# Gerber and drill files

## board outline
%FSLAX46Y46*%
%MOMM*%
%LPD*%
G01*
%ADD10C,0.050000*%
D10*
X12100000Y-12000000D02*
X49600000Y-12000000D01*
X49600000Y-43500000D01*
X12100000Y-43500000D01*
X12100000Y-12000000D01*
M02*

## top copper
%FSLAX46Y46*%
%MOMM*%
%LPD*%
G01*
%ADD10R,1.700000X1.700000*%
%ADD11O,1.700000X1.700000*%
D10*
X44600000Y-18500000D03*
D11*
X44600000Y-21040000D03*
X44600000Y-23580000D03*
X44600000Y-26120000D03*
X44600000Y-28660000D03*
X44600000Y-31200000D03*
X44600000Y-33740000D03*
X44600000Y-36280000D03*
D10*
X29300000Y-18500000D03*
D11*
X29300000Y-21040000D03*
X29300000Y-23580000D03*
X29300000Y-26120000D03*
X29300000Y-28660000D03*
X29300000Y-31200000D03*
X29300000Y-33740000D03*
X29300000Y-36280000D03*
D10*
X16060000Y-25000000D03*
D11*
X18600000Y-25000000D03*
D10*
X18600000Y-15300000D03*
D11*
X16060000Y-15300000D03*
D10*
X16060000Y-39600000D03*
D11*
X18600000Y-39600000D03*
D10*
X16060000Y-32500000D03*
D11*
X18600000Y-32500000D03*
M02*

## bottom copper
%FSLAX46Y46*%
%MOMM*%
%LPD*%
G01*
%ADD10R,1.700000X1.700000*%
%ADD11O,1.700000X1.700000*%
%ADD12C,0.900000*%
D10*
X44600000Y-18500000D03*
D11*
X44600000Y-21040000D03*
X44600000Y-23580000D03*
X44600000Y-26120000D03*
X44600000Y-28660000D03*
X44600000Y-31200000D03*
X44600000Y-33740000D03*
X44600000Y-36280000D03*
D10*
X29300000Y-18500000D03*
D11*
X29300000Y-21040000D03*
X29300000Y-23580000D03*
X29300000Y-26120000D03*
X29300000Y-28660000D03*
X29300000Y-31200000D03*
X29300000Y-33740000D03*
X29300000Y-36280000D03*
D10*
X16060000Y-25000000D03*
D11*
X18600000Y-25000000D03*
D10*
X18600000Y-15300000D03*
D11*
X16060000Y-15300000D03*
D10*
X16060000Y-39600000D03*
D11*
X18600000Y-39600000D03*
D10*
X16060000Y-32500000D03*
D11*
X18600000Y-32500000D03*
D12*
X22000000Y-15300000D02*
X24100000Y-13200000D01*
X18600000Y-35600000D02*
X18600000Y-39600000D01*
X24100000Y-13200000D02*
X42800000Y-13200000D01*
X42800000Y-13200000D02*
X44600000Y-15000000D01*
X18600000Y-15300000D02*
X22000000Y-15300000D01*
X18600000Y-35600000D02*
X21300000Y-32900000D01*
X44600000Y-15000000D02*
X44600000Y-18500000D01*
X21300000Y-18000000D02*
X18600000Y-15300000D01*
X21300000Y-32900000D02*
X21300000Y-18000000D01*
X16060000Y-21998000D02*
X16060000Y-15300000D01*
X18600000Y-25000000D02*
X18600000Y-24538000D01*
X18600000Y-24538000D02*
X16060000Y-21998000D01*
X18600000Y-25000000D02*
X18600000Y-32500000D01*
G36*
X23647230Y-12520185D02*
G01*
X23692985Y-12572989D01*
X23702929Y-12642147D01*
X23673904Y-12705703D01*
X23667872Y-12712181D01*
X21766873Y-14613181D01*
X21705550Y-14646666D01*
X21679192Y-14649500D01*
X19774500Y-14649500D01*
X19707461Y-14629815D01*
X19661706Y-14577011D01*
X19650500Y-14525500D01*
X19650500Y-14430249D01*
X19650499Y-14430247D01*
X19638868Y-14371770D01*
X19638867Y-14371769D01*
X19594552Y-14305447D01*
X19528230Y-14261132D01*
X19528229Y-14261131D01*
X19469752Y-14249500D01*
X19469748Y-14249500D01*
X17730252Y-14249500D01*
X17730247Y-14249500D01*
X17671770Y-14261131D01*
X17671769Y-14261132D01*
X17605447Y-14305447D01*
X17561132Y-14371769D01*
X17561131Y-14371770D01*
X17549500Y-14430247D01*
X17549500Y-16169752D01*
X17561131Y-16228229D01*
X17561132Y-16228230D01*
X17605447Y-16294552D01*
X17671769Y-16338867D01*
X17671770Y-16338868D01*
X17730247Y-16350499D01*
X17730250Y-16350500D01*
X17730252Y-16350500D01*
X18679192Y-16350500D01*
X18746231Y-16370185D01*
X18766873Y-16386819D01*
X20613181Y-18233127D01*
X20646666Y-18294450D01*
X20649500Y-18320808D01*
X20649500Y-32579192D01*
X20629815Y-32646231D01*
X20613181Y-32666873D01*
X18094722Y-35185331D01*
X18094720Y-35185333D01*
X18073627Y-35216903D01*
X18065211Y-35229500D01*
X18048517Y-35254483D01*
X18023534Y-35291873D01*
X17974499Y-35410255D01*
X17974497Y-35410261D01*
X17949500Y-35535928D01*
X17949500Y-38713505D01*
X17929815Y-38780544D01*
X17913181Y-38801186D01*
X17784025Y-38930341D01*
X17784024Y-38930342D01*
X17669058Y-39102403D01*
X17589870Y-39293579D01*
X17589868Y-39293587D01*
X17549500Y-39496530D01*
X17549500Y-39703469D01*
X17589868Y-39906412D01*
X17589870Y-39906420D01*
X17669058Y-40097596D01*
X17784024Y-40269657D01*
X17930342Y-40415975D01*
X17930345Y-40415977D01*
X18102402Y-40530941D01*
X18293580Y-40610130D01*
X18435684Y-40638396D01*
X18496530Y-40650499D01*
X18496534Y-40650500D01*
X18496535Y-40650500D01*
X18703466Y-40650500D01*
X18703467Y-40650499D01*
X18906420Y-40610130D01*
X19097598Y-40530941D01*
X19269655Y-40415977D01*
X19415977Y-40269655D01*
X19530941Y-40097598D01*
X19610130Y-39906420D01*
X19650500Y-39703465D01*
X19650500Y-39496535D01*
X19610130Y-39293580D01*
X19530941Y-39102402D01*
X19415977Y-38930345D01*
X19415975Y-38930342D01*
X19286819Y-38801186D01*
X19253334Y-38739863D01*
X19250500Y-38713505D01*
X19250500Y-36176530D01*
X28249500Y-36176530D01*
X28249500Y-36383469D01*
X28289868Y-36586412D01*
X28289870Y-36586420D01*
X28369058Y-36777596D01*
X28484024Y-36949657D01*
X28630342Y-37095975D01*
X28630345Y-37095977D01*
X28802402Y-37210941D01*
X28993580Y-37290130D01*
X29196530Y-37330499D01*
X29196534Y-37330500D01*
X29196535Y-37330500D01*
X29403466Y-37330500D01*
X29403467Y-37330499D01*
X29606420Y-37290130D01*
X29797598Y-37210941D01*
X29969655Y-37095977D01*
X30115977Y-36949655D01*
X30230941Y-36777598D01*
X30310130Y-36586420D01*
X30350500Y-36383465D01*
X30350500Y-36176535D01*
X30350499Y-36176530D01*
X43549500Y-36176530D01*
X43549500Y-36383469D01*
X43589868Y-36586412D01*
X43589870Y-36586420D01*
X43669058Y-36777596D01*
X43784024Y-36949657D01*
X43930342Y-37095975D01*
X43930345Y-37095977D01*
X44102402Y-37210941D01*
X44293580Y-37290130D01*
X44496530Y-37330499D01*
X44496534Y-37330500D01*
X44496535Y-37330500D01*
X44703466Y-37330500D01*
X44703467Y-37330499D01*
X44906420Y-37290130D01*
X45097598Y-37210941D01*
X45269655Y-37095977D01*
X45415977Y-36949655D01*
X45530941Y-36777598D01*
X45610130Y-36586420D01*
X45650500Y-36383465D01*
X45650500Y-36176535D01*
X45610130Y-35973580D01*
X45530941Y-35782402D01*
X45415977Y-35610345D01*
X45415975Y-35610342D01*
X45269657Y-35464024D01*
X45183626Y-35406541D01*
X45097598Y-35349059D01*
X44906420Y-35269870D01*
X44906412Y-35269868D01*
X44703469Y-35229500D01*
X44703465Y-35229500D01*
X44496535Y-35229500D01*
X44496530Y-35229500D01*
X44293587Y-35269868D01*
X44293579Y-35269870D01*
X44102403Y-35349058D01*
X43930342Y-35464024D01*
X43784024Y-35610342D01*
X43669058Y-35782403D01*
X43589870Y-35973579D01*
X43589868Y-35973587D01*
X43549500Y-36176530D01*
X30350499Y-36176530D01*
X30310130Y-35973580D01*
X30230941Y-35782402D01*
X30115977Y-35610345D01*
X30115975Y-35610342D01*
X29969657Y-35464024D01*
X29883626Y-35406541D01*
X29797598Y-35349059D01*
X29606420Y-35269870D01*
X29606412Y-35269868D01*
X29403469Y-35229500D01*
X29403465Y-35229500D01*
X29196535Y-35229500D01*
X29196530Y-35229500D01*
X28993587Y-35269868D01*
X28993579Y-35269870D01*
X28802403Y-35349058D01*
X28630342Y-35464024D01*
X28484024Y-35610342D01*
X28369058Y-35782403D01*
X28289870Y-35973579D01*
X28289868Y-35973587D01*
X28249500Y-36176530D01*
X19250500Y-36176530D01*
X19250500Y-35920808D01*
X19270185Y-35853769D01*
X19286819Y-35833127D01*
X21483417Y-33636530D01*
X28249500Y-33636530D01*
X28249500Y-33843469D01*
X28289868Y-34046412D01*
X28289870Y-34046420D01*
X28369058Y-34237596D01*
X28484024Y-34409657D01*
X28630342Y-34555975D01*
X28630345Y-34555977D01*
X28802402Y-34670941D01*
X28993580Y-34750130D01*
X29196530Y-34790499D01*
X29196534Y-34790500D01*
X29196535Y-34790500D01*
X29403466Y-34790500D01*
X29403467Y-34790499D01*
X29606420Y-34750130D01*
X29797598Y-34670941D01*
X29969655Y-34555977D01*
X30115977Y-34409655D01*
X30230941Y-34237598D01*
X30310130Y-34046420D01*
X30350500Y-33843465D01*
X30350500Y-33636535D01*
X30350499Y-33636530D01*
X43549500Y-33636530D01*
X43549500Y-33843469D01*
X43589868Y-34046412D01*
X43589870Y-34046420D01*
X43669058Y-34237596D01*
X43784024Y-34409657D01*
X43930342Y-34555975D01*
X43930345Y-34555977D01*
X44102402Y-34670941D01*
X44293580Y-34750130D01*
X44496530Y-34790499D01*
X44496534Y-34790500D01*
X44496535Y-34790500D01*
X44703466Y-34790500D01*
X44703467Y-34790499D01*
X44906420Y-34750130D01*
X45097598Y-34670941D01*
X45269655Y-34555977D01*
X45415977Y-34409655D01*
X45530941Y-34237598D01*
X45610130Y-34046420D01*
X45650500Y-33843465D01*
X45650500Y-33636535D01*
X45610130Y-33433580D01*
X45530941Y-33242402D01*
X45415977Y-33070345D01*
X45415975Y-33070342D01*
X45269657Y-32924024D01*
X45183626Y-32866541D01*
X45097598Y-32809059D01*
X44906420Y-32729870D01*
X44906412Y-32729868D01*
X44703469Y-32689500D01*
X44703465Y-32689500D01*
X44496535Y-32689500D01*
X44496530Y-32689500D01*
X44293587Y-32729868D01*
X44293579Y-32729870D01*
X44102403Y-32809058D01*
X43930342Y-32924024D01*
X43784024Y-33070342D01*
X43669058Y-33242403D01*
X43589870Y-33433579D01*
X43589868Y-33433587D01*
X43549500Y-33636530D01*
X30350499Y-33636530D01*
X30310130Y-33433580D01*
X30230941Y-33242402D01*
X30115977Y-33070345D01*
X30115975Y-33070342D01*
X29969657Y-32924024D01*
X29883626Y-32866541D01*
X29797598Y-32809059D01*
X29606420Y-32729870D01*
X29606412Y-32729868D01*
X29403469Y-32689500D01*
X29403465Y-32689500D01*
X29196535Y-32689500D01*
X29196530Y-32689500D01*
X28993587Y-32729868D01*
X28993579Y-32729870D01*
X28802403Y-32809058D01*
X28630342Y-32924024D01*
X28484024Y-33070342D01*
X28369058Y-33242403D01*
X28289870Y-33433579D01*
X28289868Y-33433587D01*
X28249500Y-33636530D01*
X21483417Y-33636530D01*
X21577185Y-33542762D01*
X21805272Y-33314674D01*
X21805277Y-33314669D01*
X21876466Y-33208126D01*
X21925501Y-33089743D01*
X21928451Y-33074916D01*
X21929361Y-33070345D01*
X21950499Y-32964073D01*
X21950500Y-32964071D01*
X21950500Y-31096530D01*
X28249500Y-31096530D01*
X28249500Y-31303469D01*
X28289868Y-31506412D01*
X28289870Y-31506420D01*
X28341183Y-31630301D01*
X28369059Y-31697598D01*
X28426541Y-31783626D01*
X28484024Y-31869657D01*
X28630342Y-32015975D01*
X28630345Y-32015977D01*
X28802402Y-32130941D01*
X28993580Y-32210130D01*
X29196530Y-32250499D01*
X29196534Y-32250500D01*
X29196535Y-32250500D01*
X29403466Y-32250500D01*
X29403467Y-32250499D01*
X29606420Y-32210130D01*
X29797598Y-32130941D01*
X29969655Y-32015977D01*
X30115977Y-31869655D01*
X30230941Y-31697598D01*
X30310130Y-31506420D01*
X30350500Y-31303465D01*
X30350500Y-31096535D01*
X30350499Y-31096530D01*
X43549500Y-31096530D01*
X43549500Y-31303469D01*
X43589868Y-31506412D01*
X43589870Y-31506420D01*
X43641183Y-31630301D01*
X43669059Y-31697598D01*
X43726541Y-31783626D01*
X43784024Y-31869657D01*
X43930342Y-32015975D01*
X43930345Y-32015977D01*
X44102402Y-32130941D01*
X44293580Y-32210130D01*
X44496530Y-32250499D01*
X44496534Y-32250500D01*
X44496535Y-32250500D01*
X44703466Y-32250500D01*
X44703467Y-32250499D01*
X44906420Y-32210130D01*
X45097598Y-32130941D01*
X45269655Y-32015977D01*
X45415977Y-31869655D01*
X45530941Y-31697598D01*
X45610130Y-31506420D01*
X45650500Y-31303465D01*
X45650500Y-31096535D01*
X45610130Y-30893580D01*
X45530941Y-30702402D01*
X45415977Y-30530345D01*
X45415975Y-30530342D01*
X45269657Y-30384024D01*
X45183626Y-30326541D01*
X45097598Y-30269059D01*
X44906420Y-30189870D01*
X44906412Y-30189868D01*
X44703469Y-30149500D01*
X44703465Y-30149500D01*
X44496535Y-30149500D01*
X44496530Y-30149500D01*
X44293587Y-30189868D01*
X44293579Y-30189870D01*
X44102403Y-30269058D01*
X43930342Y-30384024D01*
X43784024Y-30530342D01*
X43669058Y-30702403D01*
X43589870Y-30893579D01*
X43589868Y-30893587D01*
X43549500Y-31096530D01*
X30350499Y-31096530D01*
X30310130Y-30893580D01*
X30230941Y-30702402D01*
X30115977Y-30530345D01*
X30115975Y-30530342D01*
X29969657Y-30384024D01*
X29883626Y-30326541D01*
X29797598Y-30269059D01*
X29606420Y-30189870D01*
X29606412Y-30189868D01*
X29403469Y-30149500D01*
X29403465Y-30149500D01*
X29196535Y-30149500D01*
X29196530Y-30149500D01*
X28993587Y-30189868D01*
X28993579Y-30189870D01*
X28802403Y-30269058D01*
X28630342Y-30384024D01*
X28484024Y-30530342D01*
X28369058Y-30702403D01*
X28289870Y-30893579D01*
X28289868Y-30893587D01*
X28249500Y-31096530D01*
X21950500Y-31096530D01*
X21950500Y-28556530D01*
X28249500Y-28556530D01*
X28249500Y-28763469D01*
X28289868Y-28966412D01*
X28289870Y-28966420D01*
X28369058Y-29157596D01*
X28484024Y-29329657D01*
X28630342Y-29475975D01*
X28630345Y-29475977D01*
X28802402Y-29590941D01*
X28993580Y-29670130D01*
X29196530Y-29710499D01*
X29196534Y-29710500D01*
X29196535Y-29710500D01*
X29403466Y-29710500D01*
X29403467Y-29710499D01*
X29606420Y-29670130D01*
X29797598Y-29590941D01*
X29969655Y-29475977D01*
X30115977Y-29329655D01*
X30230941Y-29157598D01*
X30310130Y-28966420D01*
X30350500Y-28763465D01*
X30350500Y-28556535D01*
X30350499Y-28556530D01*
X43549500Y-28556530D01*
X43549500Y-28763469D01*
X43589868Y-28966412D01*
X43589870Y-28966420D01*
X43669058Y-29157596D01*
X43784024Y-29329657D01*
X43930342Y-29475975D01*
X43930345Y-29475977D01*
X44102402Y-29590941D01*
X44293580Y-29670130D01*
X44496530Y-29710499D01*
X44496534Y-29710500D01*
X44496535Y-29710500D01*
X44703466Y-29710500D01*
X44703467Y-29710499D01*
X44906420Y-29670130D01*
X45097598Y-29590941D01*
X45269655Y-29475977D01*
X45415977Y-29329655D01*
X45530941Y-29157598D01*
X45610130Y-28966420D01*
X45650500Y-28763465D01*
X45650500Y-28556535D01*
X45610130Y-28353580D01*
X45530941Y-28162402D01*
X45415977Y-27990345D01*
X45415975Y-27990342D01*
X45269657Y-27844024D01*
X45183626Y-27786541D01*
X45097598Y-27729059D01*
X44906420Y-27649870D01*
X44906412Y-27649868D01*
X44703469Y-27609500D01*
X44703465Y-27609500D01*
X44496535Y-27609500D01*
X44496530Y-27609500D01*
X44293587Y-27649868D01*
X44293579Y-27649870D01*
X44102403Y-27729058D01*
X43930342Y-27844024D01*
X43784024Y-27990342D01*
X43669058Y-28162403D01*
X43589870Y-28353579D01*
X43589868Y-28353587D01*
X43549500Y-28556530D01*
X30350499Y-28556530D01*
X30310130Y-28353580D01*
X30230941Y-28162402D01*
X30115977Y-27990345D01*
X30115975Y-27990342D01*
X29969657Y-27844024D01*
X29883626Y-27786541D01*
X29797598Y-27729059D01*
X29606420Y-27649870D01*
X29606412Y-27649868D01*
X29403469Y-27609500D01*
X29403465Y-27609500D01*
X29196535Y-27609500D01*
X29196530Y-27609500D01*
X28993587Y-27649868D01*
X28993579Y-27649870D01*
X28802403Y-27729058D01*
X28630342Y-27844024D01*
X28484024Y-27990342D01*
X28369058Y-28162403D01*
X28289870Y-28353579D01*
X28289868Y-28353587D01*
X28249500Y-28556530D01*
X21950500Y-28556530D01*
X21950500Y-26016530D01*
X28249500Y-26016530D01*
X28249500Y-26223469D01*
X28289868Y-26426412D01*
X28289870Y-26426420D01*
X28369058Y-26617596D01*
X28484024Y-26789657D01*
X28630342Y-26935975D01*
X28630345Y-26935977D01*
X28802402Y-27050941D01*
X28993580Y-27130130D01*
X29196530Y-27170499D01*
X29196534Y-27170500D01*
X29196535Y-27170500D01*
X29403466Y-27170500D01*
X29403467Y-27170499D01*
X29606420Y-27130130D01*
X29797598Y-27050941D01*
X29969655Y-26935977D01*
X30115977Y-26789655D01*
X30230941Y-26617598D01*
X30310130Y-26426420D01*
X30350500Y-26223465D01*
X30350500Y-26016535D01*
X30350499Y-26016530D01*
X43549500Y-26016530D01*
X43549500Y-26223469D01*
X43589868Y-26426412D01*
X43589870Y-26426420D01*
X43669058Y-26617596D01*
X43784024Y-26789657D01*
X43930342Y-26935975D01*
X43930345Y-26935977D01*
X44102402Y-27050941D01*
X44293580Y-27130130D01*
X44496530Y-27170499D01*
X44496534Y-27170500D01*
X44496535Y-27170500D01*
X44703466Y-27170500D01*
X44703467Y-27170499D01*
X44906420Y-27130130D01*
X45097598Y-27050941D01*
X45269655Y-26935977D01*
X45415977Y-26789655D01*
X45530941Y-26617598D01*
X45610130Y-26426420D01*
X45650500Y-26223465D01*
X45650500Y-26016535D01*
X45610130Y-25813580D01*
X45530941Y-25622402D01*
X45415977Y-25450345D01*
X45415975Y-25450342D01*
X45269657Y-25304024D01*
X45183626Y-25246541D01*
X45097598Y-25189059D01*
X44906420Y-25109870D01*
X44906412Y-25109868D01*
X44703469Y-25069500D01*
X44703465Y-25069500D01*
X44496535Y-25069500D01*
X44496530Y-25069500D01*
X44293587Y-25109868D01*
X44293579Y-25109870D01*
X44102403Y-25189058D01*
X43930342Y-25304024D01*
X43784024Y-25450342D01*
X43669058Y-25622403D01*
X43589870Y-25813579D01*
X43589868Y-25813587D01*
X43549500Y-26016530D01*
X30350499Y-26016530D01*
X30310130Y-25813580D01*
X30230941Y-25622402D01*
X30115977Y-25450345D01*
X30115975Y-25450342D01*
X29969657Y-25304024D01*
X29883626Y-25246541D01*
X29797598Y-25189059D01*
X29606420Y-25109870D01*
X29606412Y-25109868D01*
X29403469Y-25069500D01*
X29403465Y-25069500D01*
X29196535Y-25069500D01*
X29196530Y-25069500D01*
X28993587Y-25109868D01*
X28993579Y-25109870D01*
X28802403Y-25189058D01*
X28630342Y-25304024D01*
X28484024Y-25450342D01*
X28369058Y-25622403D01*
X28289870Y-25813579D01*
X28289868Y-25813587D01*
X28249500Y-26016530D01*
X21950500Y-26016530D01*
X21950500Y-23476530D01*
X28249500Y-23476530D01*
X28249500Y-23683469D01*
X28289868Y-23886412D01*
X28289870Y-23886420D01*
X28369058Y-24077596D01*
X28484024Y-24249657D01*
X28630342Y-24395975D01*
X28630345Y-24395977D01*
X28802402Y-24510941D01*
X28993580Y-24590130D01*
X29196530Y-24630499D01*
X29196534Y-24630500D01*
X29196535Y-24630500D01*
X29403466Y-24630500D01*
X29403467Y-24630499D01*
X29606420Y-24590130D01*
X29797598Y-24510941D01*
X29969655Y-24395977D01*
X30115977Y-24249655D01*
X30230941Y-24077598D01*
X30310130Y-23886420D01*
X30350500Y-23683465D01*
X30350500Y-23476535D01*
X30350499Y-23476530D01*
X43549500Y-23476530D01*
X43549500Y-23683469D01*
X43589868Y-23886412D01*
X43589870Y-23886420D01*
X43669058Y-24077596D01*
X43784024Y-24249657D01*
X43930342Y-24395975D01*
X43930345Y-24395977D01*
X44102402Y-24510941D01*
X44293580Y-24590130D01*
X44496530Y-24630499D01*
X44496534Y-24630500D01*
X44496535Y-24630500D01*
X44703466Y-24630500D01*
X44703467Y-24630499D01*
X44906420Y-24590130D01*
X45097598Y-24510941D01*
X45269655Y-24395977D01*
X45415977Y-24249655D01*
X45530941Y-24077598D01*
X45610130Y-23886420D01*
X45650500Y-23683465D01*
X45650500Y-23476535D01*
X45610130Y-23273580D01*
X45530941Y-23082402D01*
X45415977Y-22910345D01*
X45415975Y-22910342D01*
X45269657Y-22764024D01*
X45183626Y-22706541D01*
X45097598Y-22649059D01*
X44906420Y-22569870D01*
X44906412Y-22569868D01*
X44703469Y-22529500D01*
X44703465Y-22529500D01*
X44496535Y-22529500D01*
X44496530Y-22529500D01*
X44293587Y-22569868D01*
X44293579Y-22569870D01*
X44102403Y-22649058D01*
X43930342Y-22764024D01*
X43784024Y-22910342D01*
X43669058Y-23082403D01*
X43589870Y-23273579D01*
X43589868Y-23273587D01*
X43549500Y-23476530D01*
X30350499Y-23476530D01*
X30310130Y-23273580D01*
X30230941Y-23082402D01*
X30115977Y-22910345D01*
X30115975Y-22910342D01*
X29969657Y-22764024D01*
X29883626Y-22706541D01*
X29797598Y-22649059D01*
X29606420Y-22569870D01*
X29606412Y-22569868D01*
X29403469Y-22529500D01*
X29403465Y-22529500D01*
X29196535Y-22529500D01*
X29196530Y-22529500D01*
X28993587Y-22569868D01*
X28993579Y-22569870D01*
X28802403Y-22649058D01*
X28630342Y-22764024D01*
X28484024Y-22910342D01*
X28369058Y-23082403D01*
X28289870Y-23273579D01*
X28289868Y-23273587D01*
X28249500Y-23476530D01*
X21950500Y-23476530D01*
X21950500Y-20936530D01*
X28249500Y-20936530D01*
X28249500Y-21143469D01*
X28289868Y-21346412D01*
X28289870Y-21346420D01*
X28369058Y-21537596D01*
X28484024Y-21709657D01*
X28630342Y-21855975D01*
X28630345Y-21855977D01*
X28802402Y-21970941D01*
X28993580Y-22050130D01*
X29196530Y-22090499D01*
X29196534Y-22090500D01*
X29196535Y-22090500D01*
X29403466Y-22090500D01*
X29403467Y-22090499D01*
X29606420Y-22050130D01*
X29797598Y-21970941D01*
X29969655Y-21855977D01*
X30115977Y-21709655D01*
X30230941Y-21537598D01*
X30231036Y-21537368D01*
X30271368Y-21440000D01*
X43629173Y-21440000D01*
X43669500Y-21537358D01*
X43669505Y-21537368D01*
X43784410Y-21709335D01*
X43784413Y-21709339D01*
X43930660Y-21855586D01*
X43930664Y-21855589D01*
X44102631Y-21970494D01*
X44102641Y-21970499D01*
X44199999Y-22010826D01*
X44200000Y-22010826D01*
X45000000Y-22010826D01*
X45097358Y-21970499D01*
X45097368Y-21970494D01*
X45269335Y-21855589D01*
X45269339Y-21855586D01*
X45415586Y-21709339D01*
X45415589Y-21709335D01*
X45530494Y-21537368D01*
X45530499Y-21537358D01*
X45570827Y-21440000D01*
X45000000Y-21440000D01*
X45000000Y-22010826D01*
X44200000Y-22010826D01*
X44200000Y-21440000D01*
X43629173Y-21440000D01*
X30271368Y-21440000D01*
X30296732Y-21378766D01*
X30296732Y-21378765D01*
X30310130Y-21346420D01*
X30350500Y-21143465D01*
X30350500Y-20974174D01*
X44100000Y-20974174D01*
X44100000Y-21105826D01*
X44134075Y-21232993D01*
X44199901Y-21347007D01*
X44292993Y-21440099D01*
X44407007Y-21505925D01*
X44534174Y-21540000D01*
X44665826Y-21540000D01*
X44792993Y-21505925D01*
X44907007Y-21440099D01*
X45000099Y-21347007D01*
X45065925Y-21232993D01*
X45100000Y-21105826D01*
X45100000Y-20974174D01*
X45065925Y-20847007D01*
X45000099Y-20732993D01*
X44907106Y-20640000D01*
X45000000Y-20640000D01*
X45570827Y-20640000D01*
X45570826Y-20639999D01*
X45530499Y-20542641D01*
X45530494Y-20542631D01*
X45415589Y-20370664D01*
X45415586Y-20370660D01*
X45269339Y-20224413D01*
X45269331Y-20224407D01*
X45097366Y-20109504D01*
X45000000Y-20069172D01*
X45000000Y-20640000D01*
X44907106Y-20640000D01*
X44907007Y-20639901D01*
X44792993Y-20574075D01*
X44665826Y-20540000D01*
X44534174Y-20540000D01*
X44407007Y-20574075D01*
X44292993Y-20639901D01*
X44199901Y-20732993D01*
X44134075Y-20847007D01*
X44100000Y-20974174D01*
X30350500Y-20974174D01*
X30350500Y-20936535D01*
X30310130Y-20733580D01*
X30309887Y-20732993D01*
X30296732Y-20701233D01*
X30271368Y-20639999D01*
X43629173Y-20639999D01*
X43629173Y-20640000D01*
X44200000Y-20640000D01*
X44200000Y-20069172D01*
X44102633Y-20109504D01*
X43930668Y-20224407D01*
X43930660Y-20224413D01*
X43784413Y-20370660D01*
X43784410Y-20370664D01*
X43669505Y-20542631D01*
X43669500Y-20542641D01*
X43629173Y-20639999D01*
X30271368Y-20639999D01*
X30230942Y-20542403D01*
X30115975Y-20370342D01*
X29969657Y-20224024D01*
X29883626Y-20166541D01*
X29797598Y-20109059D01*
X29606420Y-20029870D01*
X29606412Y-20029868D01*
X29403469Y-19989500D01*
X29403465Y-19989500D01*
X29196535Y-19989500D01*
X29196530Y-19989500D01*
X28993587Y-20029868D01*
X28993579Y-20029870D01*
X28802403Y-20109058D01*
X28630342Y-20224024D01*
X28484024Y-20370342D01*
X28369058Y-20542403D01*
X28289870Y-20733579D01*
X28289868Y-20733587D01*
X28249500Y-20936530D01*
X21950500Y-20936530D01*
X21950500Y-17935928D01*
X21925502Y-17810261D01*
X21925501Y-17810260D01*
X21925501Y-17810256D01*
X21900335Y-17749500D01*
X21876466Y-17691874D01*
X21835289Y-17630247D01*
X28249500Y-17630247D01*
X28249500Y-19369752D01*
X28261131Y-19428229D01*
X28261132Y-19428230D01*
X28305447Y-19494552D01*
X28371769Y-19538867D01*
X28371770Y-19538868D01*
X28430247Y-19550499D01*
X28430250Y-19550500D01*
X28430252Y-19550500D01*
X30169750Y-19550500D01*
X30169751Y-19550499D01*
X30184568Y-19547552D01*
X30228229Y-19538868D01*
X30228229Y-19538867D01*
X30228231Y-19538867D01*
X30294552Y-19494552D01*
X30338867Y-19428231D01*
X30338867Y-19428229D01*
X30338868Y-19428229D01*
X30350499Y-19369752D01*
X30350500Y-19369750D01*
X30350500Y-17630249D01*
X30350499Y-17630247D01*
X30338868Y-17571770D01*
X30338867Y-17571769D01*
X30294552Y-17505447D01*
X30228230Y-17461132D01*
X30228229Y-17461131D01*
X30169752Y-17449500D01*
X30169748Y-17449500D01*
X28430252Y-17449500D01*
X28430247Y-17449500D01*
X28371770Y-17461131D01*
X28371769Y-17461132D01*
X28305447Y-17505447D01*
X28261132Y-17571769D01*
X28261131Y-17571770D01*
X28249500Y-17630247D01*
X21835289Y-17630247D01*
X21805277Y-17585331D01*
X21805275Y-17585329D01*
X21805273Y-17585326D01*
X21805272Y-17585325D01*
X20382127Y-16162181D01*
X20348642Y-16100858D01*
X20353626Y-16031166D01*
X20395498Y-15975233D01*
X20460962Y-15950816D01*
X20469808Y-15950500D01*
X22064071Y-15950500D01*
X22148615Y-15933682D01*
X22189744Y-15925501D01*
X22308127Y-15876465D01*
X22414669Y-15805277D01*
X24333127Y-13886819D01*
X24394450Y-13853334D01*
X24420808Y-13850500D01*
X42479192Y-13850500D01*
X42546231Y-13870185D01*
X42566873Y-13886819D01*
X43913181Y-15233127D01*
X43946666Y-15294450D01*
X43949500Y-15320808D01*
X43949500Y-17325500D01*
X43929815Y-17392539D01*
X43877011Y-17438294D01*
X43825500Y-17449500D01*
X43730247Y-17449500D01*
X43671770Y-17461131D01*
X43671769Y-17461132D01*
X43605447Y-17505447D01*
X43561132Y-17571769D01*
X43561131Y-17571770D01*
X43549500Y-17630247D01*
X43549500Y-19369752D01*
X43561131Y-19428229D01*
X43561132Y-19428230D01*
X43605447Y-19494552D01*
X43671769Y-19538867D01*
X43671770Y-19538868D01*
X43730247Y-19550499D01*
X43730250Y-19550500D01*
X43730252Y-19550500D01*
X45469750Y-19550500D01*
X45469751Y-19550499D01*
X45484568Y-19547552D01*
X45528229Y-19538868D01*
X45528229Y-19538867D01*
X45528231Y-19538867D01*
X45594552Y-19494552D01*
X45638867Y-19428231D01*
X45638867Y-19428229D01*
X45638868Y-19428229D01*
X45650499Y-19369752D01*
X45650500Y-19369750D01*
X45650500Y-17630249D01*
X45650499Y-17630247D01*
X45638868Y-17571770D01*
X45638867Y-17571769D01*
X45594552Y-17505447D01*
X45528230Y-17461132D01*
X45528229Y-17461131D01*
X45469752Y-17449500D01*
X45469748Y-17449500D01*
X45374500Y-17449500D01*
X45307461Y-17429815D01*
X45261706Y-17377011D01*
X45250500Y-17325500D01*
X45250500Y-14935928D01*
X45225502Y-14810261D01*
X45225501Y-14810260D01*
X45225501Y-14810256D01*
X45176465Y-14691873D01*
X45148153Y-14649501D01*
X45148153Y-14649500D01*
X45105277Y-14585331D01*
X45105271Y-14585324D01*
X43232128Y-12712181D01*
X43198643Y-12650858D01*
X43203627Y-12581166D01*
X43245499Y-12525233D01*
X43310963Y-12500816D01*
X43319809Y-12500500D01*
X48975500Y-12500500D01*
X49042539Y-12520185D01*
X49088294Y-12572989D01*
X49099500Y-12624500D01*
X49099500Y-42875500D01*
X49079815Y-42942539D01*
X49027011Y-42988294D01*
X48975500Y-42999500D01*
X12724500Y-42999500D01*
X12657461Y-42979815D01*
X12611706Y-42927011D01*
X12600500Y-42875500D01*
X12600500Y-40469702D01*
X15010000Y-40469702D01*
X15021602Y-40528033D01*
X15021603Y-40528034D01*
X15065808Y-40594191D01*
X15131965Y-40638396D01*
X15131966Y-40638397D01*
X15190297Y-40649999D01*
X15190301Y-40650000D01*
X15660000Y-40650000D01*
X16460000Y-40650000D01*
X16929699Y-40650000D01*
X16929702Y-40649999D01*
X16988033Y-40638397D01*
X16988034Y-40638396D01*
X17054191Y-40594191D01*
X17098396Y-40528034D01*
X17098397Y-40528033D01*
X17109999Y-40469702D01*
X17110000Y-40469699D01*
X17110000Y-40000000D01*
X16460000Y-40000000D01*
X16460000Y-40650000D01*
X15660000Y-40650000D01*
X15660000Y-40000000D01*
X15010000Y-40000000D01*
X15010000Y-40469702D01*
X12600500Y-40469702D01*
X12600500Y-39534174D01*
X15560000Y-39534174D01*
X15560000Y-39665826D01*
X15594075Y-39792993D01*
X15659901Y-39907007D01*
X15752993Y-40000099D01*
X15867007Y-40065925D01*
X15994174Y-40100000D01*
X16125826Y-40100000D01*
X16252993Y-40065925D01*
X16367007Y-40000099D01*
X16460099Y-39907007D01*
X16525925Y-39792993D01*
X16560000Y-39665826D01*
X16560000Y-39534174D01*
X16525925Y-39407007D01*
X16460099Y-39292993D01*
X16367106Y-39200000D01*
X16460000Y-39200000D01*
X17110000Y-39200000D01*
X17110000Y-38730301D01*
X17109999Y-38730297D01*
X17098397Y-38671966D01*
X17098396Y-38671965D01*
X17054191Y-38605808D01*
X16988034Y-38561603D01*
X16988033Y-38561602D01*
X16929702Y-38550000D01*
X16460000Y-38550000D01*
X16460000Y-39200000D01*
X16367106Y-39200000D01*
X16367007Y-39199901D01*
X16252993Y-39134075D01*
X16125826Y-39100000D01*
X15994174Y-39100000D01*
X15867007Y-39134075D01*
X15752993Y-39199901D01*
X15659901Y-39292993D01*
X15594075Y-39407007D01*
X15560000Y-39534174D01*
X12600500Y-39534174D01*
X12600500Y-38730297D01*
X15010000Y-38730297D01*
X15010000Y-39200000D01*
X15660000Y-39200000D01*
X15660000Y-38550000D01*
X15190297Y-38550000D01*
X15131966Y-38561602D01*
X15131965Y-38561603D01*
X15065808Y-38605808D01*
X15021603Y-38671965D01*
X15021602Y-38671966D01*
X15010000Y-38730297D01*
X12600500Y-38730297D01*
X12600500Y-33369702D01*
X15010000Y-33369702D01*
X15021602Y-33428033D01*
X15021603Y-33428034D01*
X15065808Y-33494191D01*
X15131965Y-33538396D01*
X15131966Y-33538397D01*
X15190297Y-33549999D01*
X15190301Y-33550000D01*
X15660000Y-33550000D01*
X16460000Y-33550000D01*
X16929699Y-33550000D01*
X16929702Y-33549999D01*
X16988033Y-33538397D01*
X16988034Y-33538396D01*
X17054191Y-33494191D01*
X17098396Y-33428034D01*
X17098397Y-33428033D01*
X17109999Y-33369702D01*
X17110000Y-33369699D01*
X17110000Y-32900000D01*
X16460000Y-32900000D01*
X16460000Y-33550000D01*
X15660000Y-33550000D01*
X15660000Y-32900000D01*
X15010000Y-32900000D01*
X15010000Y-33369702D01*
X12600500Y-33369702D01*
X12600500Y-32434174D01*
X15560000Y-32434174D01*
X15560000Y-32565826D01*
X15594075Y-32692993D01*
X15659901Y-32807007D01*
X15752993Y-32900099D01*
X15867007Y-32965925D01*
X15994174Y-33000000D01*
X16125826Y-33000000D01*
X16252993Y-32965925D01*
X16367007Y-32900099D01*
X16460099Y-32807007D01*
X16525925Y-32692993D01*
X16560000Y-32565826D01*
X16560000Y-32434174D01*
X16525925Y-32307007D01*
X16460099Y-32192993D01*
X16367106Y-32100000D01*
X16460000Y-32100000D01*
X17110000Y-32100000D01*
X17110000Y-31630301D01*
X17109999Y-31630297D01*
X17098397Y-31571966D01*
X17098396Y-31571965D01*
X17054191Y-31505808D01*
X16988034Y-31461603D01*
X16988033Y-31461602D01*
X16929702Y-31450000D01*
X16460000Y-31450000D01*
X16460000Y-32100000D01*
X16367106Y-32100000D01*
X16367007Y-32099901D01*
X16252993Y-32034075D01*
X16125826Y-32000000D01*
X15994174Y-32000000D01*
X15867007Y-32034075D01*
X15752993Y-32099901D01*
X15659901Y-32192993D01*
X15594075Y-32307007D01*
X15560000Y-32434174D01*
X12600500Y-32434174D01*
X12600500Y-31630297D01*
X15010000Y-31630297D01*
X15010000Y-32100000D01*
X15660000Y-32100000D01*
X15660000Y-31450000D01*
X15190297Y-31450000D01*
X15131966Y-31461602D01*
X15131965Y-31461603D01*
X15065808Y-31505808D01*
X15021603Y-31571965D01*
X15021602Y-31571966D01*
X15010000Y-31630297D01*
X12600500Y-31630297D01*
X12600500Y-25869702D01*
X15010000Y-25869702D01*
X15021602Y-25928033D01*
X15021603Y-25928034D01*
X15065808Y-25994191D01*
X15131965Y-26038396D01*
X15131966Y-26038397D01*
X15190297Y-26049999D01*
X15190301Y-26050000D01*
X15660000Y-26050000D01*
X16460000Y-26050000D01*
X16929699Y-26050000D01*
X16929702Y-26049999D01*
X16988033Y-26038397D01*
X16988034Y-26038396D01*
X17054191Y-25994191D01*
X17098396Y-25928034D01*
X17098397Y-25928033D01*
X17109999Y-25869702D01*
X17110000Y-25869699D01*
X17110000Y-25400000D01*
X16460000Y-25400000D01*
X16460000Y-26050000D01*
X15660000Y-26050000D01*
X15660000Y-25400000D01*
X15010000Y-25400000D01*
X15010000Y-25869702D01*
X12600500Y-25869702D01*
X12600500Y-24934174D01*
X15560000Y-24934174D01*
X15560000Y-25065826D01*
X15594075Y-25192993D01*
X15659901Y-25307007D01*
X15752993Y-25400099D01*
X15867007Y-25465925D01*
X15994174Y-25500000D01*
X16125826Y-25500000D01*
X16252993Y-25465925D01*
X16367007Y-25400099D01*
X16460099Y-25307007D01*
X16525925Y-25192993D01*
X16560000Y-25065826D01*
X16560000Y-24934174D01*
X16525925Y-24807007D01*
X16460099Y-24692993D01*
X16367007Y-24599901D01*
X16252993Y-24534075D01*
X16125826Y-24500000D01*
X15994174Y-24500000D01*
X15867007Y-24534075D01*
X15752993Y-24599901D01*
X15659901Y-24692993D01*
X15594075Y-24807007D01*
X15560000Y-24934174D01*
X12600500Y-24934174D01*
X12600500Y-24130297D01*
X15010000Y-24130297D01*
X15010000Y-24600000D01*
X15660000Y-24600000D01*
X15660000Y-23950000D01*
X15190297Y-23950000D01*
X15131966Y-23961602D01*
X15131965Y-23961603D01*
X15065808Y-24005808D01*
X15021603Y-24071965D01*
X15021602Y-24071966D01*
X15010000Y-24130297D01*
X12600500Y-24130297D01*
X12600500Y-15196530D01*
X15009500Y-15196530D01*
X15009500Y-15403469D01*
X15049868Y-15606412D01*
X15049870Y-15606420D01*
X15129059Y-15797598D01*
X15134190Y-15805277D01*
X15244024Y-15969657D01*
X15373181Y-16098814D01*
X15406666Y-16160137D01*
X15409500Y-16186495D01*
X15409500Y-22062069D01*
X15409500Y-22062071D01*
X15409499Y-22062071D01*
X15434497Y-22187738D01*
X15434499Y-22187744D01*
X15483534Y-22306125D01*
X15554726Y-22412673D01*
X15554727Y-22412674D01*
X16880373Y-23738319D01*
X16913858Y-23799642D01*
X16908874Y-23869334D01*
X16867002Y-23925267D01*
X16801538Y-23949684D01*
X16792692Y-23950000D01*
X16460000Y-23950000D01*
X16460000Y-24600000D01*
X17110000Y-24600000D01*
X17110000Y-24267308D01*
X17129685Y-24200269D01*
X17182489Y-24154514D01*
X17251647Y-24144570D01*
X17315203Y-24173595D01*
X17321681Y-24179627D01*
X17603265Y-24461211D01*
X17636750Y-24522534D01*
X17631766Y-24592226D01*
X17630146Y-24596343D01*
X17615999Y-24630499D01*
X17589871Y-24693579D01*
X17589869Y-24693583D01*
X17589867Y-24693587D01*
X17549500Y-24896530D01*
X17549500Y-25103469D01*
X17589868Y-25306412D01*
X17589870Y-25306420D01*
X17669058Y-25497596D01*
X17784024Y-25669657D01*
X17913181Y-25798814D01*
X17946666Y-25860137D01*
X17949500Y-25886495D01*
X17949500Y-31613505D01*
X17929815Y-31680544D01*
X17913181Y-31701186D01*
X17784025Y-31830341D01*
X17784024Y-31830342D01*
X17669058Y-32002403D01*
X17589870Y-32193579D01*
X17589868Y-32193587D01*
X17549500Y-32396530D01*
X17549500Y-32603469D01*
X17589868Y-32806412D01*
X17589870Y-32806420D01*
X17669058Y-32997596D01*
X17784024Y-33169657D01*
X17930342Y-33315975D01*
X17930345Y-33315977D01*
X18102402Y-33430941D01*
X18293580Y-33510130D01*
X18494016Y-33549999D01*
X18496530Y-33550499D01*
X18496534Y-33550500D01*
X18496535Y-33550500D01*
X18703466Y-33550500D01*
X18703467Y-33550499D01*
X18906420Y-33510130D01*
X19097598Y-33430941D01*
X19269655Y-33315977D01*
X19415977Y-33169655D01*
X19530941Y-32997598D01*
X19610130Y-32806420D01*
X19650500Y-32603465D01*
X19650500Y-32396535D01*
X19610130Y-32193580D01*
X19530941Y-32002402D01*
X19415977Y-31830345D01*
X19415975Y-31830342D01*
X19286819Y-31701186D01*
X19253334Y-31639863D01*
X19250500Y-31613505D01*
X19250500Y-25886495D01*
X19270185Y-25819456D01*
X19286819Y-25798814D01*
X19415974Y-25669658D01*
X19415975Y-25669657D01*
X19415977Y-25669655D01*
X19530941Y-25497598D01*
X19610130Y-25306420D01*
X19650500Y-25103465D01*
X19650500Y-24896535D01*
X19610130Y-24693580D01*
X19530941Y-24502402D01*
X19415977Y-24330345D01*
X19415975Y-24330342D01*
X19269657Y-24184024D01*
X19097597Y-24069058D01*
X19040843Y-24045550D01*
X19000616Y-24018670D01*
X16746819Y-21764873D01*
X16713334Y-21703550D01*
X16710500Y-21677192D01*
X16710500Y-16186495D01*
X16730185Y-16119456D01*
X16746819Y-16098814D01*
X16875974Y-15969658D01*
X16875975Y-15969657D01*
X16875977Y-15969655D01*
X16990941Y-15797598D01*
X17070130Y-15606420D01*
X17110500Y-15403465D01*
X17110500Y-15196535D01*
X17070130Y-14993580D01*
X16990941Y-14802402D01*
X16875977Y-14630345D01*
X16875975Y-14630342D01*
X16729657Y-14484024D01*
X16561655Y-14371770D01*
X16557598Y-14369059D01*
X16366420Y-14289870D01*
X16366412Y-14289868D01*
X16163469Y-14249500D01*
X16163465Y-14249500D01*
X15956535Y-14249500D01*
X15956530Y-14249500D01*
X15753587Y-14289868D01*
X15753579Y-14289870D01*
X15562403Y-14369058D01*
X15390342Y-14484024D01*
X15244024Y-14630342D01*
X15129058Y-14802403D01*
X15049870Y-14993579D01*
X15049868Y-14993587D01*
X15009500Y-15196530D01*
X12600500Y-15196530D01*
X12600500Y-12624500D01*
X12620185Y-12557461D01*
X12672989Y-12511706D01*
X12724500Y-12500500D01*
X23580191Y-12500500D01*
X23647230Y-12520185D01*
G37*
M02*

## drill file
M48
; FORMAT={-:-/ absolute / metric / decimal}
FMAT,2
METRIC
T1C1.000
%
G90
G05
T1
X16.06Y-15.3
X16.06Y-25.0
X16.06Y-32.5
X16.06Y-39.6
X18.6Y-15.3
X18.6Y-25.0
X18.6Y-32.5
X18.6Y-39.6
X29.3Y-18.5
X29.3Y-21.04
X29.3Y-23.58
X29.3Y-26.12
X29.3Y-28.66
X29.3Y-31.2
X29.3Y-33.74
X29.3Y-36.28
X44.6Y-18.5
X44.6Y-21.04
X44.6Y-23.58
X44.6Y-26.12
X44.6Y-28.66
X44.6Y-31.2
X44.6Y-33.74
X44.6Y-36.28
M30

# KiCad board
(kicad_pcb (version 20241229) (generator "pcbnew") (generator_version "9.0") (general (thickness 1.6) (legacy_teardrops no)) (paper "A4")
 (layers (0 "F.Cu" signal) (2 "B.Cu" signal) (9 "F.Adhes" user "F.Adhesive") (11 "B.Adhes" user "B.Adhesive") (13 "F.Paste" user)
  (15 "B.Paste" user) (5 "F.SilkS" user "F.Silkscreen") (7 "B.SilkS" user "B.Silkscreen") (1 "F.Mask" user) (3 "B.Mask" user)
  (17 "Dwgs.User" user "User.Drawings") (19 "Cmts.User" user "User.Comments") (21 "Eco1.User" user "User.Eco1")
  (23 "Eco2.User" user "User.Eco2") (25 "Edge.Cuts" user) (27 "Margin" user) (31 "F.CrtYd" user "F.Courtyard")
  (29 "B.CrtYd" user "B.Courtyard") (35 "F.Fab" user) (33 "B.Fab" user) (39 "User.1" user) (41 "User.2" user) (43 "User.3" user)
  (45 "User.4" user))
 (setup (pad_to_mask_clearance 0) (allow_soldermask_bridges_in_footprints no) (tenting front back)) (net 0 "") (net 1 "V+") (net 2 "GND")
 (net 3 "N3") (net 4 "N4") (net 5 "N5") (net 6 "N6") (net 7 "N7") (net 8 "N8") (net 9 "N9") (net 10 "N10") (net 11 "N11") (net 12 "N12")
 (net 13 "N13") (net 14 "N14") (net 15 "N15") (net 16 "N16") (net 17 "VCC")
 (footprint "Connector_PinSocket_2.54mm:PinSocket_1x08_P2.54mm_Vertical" (layer "F.Cu") (at 44.6 18.5)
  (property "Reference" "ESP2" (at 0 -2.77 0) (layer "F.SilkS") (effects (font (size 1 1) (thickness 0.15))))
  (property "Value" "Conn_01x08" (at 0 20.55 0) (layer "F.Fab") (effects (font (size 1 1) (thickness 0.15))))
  (pad "1" thru_hole rect (at 0 0) (size 1.7 1.7) (drill 1) (layers "*.Cu" "*.Mask") (remove_unused_layers no) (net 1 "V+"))
  (pad "2" thru_hole oval (at 0 2.54) (size 1.7 1.7) (drill 1) (layers "*.Cu" "*.Mask") (remove_unused_layers no) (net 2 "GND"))
  (pad "3" thru_hole oval (at 0 5.08) (size 1.7 1.7) (drill 1) (layers "*.Cu" "*.Mask") (remove_unused_layers no) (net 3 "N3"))
  (pad "4" thru_hole oval (at 0 7.62) (size 1.7 1.7) (drill 1) (layers "*.Cu" "*.Mask") (remove_unused_layers no) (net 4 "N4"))
  (pad "5" thru_hole oval (at 0 10.16) (size 1.7 1.7) (drill 1) (layers "*.Cu" "*.Mask") (remove_unused_layers no) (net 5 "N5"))
  (pad "6" thru_hole oval (at 0 12.7) (size 1.7 1.7) (drill 1) (layers "*.Cu" "*.Mask") (remove_unused_layers no) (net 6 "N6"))
  (pad "7" thru_hole oval (at 0 15.24) (size 1.7 1.7) (drill 1) (layers "*.Cu" "*.Mask") (remove_unused_layers no) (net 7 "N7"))
  (pad "8" thru_hole oval (at 0 17.78) (size 1.7 1.7) (drill 1) (layers "*.Cu" "*.Mask") (remove_unused_layers no) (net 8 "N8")))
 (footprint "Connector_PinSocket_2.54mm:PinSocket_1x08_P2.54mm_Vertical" (layer "F.Cu") (at 29.3 18.5)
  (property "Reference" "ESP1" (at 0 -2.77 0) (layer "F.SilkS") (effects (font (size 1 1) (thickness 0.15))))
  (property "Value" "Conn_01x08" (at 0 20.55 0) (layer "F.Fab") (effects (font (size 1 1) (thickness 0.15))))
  (pad "1" thru_hole rect (at 0 0) (size 1.7 1.7) (drill 1) (layers "*.Cu" "*.Mask") (remove_unused_layers no) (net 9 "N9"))
  (pad "2" thru_hole oval (at 0 2.54) (size 1.7 1.7) (drill 1) (layers "*.Cu" "*.Mask") (remove_unused_layers no) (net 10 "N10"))
  (pad "3" thru_hole oval (at 0 5.08) (size 1.7 1.7) (drill 1) (layers "*.Cu" "*.Mask") (remove_unused_layers no) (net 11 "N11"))
  (pad "4" thru_hole oval (at 0 7.62) (size 1.7 1.7) (drill 1) (layers "*.Cu" "*.Mask") (remove_unused_layers no) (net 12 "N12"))
  (pad "5" thru_hole oval (at 0 10.16) (size 1.7 1.7) (drill 1) (layers "*.Cu" "*.Mask") (remove_unused_layers no) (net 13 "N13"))
  (pad "6" thru_hole oval (at 0 12.7) (size 1.7 1.7) (drill 1) (layers "*.Cu" "*.Mask") (remove_unused_layers no) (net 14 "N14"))
  (pad "7" thru_hole oval (at 0 15.24) (size 1.7 1.7) (drill 1) (layers "*.Cu" "*.Mask") (remove_unused_layers no) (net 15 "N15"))
  (pad "8" thru_hole oval (at 0 17.78) (size 1.7 1.7) (drill 1) (layers "*.Cu" "*.Mask") (remove_unused_layers no) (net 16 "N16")))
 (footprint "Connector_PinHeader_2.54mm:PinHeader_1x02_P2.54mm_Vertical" (layer "F.Cu") (at 16.06 25 90)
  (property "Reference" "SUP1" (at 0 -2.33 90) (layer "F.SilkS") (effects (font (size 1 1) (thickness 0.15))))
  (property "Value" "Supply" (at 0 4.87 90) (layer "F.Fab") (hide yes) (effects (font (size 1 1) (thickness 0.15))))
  (pad "1" thru_hole rect (at 0 0 90) (size 1.7 1.7) (drill 1) (layers "*.Cu" "*.Mask") (remove_unused_layers no) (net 2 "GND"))
  (pad "2" thru_hole oval (at 0 2.54 90) (size 1.7 1.7) (drill 1) (layers "*.Cu" "*.Mask") (remove_unused_layers no) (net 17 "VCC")))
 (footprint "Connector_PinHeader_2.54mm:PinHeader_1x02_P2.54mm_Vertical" (layer "F.Cu") (at 18.6 15.3 -90)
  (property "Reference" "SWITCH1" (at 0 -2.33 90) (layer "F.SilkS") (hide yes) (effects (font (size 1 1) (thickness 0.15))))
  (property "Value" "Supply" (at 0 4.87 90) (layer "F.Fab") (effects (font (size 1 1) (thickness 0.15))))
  (pad "1" thru_hole rect (at 0 0 270) (size 1.7 1.7) (drill 1) (layers "*.Cu" "*.Mask") (remove_unused_layers no) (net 1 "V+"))
  (pad "2" thru_hole oval (at 0 2.54 270) (size 1.7 1.7) (drill 1) (layers "*.Cu" "*.Mask") (remove_unused_layers no) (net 17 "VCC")))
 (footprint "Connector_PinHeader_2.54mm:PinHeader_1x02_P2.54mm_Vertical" (layer "F.Cu") (at 16.06 39.6 90)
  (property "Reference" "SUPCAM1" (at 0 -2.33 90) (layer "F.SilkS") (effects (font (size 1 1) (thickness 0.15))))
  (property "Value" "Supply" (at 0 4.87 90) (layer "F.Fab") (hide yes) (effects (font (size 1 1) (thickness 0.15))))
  (pad "1" thru_hole rect (at 0 0 90) (size 1.7 1.7) (drill 1) (layers "*.Cu" "*.Mask") (remove_unused_layers no) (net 2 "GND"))
  (pad "2" thru_hole oval (at 0 2.54 90) (size 1.7 1.7) (drill 1) (layers "*.Cu" "*.Mask") (remove_unused_layers no) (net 1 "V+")))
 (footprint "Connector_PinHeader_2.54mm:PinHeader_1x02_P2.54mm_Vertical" (layer "F.Cu") (at 16.06 32.5 90)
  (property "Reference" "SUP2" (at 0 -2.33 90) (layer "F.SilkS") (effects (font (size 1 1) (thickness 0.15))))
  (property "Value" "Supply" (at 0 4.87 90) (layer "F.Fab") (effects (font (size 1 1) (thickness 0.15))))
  (pad "1" thru_hole rect (at 0 0 90) (size 1.7 1.7) (drill 1) (layers "*.Cu" "*.Mask") (remove_unused_layers no) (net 2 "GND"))
  (pad "2" thru_hole oval (at 0 2.54 90) (size 1.7 1.7) (drill 1) (layers "*.Cu" "*.Mask") (remove_unused_layers no) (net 17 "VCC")))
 (gr_rect (start 12.1 12) (end 49.6 43.5) (stroke (width 0.05) (type solid)) (fill no) (layer "Edge.Cuts"))
 (segment (start 22 15.3) (end 24.1 13.2) (width 0.9) (layer "B.Cu") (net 1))
 (segment (start 18.6 35.6) (end 18.6 39.6) (width 0.9) (layer "B.Cu") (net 1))
 (segment (start 24.1 13.2) (end 42.8 13.2) (width 0.9) (layer "B.Cu") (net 1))
 (segment (start 42.8 13.2) (end 44.6 15) (width 0.9) (layer "B.Cu") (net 1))
 (segment (start 18.6 15.3) (end 22 15.3) (width 0.9) (layer "B.Cu") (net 1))
 (segment (start 18.6 35.6) (end 21.3 32.9) (width 0.9) (layer "B.Cu") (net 1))
 (segment (start 44.6 15) (end 44.6 18.5) (width 0.9) (layer "B.Cu") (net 1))
 (segment (start 21.3 18) (end 18.6 15.3) (width 0.9) (layer "B.Cu") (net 1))
 (segment (start 21.3 32.9) (end 21.3 18) (width 0.9) (layer "B.Cu") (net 1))
 (segment (start 16.06 21.998) (end 16.06 15.3) (width 0.9) (layer "B.Cu") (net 17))
 (segment (start 18.6 25) (end 18.6 24.538) (width 0.9) (layer "B.Cu") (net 17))
 (segment (start 18.6 24.538) (end 16.06 21.998) (width 0.9) (layer "B.Cu") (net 17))
 (segment (start 18.6 25) (end 18.6 32.5) (width 0.9) (layer "B.Cu") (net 17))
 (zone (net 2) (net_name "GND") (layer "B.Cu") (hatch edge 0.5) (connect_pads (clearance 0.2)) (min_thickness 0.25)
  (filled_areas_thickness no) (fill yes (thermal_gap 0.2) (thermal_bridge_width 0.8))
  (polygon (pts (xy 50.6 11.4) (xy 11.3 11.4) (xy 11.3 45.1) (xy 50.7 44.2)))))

